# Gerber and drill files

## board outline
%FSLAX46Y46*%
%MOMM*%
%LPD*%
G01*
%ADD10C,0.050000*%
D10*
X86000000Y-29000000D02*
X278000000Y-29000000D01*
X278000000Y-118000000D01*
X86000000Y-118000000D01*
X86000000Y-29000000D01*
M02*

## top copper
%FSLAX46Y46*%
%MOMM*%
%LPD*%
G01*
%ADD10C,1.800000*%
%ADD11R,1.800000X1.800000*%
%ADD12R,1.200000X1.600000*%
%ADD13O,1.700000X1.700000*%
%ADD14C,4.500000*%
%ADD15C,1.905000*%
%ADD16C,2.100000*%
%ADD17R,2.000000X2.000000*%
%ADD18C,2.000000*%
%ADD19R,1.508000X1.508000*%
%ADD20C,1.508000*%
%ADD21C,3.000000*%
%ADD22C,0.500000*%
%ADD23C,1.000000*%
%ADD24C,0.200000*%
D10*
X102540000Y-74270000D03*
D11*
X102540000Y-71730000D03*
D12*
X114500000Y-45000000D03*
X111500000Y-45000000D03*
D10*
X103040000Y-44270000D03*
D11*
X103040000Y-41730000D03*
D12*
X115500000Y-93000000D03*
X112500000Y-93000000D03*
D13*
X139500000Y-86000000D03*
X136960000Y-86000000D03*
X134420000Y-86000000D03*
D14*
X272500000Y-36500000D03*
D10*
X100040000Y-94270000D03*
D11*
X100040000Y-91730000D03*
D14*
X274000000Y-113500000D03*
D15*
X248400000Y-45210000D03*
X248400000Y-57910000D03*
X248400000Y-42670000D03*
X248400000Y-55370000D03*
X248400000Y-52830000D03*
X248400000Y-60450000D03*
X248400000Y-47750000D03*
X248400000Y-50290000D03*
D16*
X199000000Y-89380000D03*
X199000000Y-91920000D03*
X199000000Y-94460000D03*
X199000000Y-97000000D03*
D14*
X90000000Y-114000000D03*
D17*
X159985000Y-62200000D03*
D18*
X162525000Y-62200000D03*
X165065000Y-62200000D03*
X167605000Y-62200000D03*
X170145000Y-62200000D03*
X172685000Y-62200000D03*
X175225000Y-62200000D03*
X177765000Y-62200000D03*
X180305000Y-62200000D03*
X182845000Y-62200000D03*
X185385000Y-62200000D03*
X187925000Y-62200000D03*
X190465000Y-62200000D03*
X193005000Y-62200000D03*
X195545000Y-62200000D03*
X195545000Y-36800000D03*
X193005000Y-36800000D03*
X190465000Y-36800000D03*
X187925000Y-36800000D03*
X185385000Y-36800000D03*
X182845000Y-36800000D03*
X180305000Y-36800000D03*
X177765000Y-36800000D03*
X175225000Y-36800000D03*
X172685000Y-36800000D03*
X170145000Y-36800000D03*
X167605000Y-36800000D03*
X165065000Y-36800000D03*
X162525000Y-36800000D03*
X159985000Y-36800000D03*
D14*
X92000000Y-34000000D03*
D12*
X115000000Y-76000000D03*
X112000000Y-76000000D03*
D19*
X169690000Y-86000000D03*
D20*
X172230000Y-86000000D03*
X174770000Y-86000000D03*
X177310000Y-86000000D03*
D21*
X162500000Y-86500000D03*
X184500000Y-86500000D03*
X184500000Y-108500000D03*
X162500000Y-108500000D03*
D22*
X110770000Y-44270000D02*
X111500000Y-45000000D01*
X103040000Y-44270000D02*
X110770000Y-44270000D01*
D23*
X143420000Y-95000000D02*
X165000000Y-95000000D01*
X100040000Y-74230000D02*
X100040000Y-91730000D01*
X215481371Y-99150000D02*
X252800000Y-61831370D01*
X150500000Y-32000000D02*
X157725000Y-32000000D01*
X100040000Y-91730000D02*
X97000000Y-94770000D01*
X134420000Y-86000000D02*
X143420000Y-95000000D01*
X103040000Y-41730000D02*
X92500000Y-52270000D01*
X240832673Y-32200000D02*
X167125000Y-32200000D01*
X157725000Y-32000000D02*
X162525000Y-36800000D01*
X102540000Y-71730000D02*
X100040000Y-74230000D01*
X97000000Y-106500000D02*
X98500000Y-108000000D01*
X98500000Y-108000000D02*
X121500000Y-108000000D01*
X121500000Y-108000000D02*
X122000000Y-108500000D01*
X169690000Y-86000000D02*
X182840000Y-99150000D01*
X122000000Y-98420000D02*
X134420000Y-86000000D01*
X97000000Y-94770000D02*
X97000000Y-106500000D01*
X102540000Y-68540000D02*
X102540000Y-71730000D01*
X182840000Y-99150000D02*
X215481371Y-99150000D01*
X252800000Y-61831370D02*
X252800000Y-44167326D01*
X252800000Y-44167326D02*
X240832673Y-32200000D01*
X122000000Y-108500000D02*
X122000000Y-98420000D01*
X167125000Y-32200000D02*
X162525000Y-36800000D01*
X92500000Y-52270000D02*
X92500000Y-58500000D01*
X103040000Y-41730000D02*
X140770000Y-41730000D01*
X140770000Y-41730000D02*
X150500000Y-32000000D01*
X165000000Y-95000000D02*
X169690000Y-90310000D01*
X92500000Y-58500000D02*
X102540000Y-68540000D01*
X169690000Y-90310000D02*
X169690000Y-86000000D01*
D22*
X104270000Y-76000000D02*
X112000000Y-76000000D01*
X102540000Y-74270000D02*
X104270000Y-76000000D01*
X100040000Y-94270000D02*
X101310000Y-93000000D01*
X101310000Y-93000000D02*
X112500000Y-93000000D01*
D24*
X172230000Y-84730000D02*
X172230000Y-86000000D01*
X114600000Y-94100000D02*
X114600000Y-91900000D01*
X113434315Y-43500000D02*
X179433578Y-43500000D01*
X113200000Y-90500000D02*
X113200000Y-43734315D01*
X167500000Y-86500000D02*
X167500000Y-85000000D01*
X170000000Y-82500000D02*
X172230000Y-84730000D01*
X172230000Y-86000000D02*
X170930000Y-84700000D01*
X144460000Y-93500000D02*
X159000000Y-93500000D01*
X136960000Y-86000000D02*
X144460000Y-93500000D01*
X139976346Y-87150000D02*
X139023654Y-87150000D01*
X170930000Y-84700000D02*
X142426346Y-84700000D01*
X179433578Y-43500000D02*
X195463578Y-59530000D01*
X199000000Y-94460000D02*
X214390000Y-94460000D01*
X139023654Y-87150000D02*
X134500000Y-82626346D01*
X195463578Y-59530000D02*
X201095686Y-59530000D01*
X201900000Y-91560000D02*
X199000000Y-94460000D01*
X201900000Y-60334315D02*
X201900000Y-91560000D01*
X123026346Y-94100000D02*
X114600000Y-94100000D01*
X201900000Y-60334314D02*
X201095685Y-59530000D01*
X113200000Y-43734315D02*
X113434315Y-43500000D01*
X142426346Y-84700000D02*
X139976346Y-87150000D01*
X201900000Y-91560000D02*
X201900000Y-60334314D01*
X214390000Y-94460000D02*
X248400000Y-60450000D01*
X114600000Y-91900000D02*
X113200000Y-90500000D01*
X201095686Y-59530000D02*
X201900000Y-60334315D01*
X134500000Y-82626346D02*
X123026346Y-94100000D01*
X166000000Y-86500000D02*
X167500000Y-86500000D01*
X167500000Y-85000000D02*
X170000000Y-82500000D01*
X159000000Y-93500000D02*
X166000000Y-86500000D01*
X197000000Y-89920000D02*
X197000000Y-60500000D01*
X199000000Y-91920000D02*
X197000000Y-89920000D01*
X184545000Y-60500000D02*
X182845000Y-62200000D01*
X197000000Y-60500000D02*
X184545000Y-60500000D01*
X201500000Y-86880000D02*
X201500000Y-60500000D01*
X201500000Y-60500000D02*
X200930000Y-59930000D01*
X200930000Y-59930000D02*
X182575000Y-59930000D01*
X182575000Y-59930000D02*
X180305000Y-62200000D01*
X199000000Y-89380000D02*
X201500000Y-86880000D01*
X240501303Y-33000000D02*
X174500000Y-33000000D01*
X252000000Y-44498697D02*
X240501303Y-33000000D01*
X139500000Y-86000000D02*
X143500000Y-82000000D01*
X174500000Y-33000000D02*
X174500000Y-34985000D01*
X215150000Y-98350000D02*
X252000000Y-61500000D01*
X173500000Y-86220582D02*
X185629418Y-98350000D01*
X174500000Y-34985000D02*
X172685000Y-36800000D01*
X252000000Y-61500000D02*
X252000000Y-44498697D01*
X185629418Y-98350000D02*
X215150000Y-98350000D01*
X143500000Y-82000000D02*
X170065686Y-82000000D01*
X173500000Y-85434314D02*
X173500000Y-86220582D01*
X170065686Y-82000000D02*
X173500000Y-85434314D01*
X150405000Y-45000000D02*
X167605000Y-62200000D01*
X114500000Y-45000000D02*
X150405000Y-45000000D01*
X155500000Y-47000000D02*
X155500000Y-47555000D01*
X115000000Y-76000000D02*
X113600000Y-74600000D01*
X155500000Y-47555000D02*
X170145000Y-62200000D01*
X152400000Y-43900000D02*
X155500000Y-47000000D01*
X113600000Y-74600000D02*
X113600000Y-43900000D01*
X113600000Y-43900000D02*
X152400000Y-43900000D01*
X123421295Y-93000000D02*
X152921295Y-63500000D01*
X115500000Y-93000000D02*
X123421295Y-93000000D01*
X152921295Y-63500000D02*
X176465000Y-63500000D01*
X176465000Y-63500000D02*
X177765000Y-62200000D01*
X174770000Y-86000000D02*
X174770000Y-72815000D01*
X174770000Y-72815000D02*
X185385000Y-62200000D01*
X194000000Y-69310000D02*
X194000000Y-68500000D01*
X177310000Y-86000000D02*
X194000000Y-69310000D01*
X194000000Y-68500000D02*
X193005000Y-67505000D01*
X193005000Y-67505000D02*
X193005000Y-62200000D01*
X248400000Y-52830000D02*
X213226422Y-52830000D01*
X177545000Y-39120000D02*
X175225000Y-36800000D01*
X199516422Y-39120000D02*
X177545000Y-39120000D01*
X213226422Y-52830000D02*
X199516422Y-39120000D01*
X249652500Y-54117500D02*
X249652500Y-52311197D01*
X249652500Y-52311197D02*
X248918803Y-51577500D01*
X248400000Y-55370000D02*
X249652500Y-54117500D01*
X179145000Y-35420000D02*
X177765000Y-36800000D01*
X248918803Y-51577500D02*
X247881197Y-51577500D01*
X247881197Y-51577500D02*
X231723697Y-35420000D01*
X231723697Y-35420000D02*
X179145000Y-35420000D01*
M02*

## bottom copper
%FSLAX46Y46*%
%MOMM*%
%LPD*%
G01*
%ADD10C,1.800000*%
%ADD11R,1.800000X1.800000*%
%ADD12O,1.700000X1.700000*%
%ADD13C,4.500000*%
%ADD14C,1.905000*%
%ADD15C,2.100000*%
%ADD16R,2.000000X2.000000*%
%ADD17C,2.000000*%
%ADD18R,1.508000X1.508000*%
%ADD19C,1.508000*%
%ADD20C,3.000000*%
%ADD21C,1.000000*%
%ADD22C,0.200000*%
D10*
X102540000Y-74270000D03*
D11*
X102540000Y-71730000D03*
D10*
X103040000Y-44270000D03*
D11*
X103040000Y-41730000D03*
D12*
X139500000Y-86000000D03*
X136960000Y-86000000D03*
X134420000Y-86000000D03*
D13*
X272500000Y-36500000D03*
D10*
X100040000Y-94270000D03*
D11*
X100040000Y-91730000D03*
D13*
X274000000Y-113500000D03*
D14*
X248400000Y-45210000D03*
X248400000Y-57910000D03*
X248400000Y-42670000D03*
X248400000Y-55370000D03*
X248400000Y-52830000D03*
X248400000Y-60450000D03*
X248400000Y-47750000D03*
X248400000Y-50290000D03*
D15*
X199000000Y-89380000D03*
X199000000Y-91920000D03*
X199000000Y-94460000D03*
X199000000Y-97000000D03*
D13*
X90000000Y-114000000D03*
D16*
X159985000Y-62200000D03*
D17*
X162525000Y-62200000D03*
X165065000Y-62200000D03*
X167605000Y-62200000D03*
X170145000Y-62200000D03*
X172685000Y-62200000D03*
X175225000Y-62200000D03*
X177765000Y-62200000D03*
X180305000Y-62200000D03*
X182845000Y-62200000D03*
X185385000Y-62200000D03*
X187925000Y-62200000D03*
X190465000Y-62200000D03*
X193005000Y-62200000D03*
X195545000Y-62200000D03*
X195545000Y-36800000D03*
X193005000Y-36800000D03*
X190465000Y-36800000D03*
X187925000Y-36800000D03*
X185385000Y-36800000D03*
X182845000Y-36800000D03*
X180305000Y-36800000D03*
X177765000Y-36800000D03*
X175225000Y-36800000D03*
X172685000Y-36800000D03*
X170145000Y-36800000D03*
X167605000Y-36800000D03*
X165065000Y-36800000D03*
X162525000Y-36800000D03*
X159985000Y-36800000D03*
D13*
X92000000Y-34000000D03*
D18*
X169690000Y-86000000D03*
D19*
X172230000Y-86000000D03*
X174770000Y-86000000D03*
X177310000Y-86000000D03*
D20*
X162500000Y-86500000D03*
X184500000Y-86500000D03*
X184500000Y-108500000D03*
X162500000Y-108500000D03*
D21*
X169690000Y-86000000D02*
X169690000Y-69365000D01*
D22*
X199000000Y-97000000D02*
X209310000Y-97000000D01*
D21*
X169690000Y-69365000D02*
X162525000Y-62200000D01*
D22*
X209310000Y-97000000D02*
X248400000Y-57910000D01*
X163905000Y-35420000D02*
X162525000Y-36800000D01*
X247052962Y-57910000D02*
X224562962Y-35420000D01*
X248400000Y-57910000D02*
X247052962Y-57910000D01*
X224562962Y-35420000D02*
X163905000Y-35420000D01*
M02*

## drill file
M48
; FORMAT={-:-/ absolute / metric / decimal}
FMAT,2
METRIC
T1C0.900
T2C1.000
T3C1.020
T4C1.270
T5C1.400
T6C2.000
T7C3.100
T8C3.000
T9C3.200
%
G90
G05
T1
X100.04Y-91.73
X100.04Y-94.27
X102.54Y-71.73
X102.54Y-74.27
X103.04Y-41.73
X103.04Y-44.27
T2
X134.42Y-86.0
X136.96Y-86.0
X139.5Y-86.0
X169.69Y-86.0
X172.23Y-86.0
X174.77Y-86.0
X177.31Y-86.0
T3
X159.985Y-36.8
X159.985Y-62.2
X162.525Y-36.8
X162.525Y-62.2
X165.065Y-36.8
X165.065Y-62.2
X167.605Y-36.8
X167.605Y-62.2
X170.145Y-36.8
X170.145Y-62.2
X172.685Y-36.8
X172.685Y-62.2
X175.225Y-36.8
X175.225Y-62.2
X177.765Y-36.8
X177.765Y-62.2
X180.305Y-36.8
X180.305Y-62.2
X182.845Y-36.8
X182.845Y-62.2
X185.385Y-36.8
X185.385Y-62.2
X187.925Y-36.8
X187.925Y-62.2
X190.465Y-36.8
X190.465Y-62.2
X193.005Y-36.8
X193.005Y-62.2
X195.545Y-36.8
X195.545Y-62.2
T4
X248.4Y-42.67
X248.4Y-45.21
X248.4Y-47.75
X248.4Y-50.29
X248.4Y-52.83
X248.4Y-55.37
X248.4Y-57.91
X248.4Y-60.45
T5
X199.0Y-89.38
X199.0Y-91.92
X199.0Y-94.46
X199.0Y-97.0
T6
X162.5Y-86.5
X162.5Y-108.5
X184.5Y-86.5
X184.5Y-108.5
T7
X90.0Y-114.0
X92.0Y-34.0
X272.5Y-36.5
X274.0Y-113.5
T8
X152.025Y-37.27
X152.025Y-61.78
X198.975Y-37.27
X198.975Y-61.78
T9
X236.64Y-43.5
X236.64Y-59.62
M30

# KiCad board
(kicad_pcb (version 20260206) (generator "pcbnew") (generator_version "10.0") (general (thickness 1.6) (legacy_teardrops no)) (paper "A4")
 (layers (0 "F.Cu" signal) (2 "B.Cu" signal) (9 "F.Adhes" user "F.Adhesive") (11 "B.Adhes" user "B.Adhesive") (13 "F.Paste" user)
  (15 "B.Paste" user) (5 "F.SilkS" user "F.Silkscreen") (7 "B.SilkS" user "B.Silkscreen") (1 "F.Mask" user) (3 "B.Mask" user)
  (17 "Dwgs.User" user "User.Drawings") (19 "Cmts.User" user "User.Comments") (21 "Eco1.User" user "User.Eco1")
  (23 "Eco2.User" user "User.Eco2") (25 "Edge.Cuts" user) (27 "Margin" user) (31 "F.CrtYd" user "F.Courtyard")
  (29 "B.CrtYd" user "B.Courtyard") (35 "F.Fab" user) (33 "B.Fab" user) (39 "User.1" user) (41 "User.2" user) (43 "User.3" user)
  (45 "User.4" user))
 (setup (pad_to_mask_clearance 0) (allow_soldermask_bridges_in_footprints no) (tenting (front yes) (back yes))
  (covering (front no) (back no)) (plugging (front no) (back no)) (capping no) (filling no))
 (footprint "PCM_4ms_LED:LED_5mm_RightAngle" (layer "F.Cu") (at 98 73 -90)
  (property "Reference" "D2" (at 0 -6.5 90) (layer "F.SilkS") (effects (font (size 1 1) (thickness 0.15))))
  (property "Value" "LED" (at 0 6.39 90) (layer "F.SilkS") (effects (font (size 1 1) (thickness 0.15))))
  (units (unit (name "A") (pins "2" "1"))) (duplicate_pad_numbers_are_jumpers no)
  (pad "1" thru_hole circle (at 1.27 -4.54 270) (size 1.8 1.8) (drill 0.9) (layers "*.Cu" "*.Mask") (remove_unused_layers no)
   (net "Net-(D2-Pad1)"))
  (pad "2" thru_hole rect (at -1.27 -4.54 270) (size 1.8 1.8) (drill 0.9) (layers "*.Cu" "*.Mask") (remove_unused_layers no) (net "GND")))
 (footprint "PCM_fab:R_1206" (layer "F.Cu") (at 113 45 180)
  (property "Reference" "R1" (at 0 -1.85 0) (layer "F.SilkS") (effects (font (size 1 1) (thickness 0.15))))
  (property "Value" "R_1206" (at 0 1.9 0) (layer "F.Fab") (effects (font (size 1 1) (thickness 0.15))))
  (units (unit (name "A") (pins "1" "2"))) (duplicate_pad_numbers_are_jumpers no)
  (pad "1" smd rect (at -1.5 0 180) (size 1.2 1.6) (layers "F.Cu" "F.Mask" "F.Paste") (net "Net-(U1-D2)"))
  (pad "2" smd rect (at 1.5 0 180) (size 1.2 1.6) (layers "F.Cu" "F.Mask" "F.Paste") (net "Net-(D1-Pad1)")))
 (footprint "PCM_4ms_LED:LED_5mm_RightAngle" (layer "F.Cu") (at 98.5 43 -90)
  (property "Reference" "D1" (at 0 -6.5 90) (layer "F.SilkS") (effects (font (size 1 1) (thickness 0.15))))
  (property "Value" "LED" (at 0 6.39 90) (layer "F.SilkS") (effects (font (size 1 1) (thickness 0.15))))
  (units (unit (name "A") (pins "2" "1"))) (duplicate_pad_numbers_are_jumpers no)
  (pad "1" thru_hole circle (at 1.27 -4.54 270) (size 1.8 1.8) (drill 0.9) (layers "*.Cu" "*.Mask") (remove_unused_layers no)
   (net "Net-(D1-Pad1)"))
  (pad "2" thru_hole rect (at -1.27 -4.54 270) (size 1.8 1.8) (drill 0.9) (layers "*.Cu" "*.Mask") (remove_unused_layers no) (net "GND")))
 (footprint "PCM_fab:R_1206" (layer "F.Cu") (at 114 93 180)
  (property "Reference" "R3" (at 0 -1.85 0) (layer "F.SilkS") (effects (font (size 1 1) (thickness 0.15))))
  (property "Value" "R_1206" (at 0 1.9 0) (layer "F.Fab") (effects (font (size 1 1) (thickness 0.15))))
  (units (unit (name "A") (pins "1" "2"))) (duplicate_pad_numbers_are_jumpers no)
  (pad "1" smd rect (at -1.5 0 180) (size 1.2 1.6) (layers "F.Cu" "F.Mask" "F.Paste") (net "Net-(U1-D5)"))
  (pad "2" smd rect (at 1.5 0 180) (size 1.2 1.6) (layers "F.Cu" "F.Mask" "F.Paste") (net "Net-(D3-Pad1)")))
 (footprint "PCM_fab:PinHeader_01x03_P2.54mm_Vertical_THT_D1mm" (layer "F.Cu") (at 139.5 86 -90)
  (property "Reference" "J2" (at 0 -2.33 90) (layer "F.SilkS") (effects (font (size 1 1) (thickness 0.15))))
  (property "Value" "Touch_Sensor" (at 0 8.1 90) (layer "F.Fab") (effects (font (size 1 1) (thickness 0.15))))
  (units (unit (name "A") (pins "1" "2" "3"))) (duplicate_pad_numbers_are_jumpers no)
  (pad "1" thru_hole oval (at 0 0 270) (size 1.7 1.7) (drill 1) (layers "*.Cu" "*.Mask") (remove_unused_layers no) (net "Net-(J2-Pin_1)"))
  (pad "2" thru_hole oval (at 0 2.54 270) (size 1.7 1.7) (drill 1) (layers "*.Cu" "*.Mask") (remove_unused_layers no) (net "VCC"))
  (pad "3" thru_hole oval (at 0 5.08 270) (size 1.7 1.7) (drill 1) (layers "*.Cu" "*.Mask") (remove_unused_layers no) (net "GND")))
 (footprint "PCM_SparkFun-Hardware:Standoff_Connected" (layer "F.Cu") (at 272.5 36.5)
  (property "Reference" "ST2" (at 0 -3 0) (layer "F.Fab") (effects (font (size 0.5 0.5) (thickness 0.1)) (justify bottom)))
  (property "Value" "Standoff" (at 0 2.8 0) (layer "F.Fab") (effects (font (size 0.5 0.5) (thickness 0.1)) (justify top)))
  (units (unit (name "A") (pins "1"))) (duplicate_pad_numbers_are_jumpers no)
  (pad "1" thru_hole circle (at 0 0) (size 4.5 4.5) (drill 3.1) (layers "*.Cu" "*.Mask") (remove_unused_layers no)
   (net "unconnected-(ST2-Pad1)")))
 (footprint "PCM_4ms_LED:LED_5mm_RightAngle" (layer "F.Cu") (at 95.5 93 -90)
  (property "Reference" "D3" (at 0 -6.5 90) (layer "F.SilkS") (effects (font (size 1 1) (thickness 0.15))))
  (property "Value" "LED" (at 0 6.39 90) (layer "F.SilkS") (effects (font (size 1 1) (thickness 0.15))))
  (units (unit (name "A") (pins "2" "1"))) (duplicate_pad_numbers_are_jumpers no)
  (pad "1" thru_hole circle (at 1.27 -4.54 270) (size 1.8 1.8) (drill 0.9) (layers "*.Cu" "*.Mask") (remove_unused_layers no)
   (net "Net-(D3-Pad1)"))
  (pad "2" thru_hole rect (at -1.27 -4.54 270) (size 1.8 1.8) (drill 0.9) (layers "*.Cu" "*.Mask") (remove_unused_layers no) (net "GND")))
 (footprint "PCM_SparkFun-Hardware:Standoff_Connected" (layer "F.Cu") (at 274 113.5)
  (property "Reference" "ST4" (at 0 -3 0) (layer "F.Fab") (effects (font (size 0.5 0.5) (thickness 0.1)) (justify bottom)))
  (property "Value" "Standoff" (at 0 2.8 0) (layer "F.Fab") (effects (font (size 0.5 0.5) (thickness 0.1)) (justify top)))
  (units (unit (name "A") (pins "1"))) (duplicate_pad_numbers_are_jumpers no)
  (pad "1" thru_hole circle (at 0 0) (size 4.5 4.5) (drill 3.1) (layers "*.Cu" "*.Mask") (remove_unused_layers no)
   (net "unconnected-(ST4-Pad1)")))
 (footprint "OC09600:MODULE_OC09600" (layer "F.Cu") (at 242.07 51.56 180)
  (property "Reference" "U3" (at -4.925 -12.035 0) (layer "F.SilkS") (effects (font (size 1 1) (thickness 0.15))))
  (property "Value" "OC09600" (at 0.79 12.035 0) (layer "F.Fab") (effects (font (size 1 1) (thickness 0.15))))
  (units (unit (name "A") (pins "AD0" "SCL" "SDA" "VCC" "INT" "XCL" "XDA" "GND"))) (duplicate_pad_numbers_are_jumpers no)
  (pad "" np_thru_hole circle (at 5.43 -8.06 180) (size 3.2 3.2) (drill 3.2) (layers "*.Cu" "*.Mask"))
  (pad "" np_thru_hole circle (at 5.43 8.06 180) (size 3.2 3.2) (drill 3.2) (layers "*.Cu" "*.Mask"))
  (pad "AD0" thru_hole circle (at -6.33 6.35 180) (size 1.905 1.905) (drill 1.27) (layers "*.Cu" "*.Mask") (remove_unused_layers no)
   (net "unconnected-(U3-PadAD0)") (solder_mask_margin 0.102))
  (pad "GND" thru_hole circle (at -6.33 -6.35 180) (size 1.905 1.905) (drill 1.27) (layers "*.Cu" "*.Mask") (remove_unused_layers no)
   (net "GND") (solder_mask_margin 0.102))
  (pad "INT" thru_hole circle (at -6.33 8.89 180) (size 1.905 1.905) (drill 1.27) (layers "*.Cu" "*.Mask") (remove_unused_layers no)
   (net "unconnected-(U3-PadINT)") (solder_mask_margin 0.102))
  (pad "SCL" thru_hole circle (at -6.33 -3.81 180) (size 1.905 1.905) (drill 1.27) (layers "*.Cu" "*.Mask") (remove_unused_layers no)
   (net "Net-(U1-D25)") (solder_mask_margin 0.102))
  (pad "SDA" thru_hole circle (at -6.33 -1.27 180) (size 1.905 1.905) (drill 1.27) (layers "*.Cu" "*.Mask") (remove_unused_layers no)
   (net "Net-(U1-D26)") (solder_mask_margin 0.102))
  (pad "VCC" thru_hole circle (at -6.33 -8.89 180) (size 1.905 1.905) (drill 1.27) (layers "*.Cu" "*.Mask") (remove_unused_layers no)
   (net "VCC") (solder_mask_margin 0.102))
  (pad "XCL" thru_hole circle (at -6.33 3.81 180) (size 1.905 1.905) (drill 1.27) (layers "*.Cu" "*.Mask") (remove_unused_layers no)
   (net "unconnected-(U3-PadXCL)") (solder_mask_margin 0.102))
  (pad "XDA" thru_hole circle (at -6.33 1.27 180) (size 1.905 1.905) (drill 1.27) (layers "*.Cu" "*.Mask") (remove_unused_layers no)
   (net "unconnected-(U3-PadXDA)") (solder_mask_margin 0.102)))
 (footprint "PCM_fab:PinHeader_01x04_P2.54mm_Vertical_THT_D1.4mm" (layer "F.Cu") (at 199 89.38)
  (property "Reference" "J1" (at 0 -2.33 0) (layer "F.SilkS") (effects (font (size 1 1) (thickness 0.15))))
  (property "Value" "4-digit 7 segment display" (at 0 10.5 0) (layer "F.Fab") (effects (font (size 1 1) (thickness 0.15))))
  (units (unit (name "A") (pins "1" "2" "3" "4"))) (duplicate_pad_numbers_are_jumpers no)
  (pad "1" thru_hole circle (at 0 0) (size 2.1 2.1) (drill 1.4) (layers "*.Cu" "*.Mask") (remove_unused_layers no) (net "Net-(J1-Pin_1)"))
  (pad "2" thru_hole circle (at 0 2.54) (size 2.1 2.1) (drill 1.4) (layers "*.Cu" "*.Mask") (remove_unused_layers no) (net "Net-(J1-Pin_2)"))
  (pad "3" thru_hole circle (at 0 5.08) (size 2.1 2.1) (drill 1.4) (layers "*.Cu" "*.Mask") (remove_unused_layers no) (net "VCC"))
  (pad "4" thru_hole circle (at 0 7.62) (size 2.1 2.1) (drill 1.4) (layers "*.Cu" "*.Mask") (remove_unused_layers no) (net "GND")))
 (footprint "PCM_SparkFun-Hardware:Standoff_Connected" (layer "F.Cu") (at 90 114)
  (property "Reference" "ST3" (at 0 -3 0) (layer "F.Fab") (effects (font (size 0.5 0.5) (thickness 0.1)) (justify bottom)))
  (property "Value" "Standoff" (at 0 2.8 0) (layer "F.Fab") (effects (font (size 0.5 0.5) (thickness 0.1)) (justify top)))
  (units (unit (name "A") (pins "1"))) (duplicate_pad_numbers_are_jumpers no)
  (pad "1" thru_hole circle (at 0 0) (size 4.5 4.5) (drill 3.1) (layers "*.Cu" "*.Mask") (remove_unused_layers no)
   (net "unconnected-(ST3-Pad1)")))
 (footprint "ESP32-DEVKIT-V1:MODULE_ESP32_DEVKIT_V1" (layer "F.Cu") (at 175.5 49.5 90)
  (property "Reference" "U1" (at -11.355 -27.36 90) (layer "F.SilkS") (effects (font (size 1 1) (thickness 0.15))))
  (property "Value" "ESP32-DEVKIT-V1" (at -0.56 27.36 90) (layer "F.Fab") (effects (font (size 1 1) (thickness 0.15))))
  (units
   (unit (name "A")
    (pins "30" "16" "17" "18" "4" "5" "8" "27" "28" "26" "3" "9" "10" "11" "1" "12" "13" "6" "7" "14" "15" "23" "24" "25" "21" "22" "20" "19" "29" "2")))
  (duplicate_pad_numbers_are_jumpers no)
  (pad "" np_thru_hole circle (at -12.28 -23.475 90) (size 3 3) (drill 3) (layers "*.Cu" "*.Mask"))
  (pad "" np_thru_hole circle (at -12.28 23.475 90) (size 3 3) (drill 3) (layers "*.Cu" "*.Mask"))
  (pad "" np_thru_hole circle (at 12.23 -23.475 90) (size 3 3) (drill 3) (layers "*.Cu" "*.Mask"))
  (pad "" np_thru_hole circle (at 12.23 23.475 90) (size 3 3) (drill 3) (layers "*.Cu" "*.Mask"))
  (pad "1" thru_hole rect (at -12.7 -15.515 90) (size 2 2) (drill 1.02) (layers "*.Cu" "*.Mask") (remove_unused_layers no) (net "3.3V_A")
   (solder_mask_margin 0.102))
  (pad "2" thru_hole circle (at -12.7 -12.975 90) (size 2 2) (drill 1.02) (layers "*.Cu" "*.Mask") (remove_unused_layers no) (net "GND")
   (solder_mask_margin 0.102))
  (pad "3" thru_hole circle (at -12.7 -10.435 90) (size 2 2) (drill 1.02) (layers "*.Cu" "*.Mask") (remove_unused_layers no)
   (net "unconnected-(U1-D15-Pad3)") (solder_mask_margin 0.102))
  (pad "4" thru_hole circle (at -12.7 -7.895 90) (size 2 2) (drill 1.02) (layers "*.Cu" "*.Mask") (remove_unused_layers no)
   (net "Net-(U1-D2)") (solder_mask_margin 0.102))
  (pad "5" thru_hole circle (at -12.7 -5.355 90) (size 2 2) (drill 1.02) (layers "*.Cu" "*.Mask") (remove_unused_layers no)
   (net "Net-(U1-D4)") (solder_mask_margin 0.102))
  (pad "6" thru_hole circle (at -12.7 -2.815 90) (size 2 2) (drill 1.02) (layers "*.Cu" "*.Mask") (remove_unused_layers no)
   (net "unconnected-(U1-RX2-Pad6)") (solder_mask_margin 0.102))
  (pad "7" thru_hole circle (at -12.7 -0.275 90) (size 2 2) (drill 1.02) (layers "*.Cu" "*.Mask") (remove_unused_layers no)
   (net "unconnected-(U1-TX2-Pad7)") (solder_mask_margin 0.102))
  (pad "8" thru_hole circle (at -12.7 2.265 90) (size 2 2) (drill 1.02) (layers "*.Cu" "*.Mask") (remove_unused_layers no)
   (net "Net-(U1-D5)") (solder_mask_margin 0.102))
  (pad "9" thru_hole circle (at -12.7 4.805 90) (size 2 2) (drill 1.02) (layers "*.Cu" "*.Mask") (remove_unused_layers no)
   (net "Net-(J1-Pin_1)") (solder_mask_margin 0.102))
  (pad "10" thru_hole circle (at -12.7 7.345 90) (size 2 2) (drill 1.02) (layers "*.Cu" "*.Mask") (remove_unused_layers no)
   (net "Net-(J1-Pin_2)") (solder_mask_margin 0.102))
  (pad "11" thru_hole circle (at -12.7 9.885 90) (size 2 2) (drill 1.02) (layers "*.Cu" "*.Mask") (remove_unused_layers no) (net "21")
   (solder_mask_margin 0.102))
  (pad "12" thru_hole circle (at -12.7 12.425 90) (size 2 2) (drill 1.02) (layers "*.Cu" "*.Mask") (remove_unused_layers no)
   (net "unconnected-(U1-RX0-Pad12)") (solder_mask_margin 0.102))
  (pad "13" thru_hole circle (at -12.7 14.965 90) (size 2 2) (drill 1.02) (layers "*.Cu" "*.Mask") (remove_unused_layers no)
   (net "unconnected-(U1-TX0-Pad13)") (solder_mask_margin 0.102))
  (pad "14" thru_hole circle (at -12.7 17.505 90) (size 2 2) (drill 1.02) (layers "*.Cu" "*.Mask") (remove_unused_layers no) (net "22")
   (solder_mask_margin 0.102))
  (pad "15" thru_hole circle (at -12.7 20.045 90) (size 2 2) (drill 1.02) (layers "*.Cu" "*.Mask") (remove_unused_layers no)
   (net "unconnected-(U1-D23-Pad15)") (solder_mask_margin 0.102))
  (pad "16" thru_hole circle (at 12.7 20.045 90) (size 2 2) (drill 1.02) (layers "*.Cu" "*.Mask") (remove_unused_layers no)
   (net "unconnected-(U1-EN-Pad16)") (solder_mask_margin 0.102))
  (pad "17" thru_hole circle (at 12.7 17.505 90) (size 2 2) (drill 1.02) (layers "*.Cu" "*.Mask") (remove_unused_layers no)
   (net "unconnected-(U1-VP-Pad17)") (solder_mask_margin 0.102))
  (pad "18" thru_hole circle (at 12.7 14.965 90) (size 2 2) (drill 1.02) (layers "*.Cu" "*.Mask") (remove_unused_layers no)
   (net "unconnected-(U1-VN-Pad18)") (solder_mask_margin 0.102))
  (pad "19" thru_hole circle (at 12.7 12.425 90) (size 2 2) (drill 1.02) (layers "*.Cu" "*.Mask") (remove_unused_layers no)
   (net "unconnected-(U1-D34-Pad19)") (solder_mask_margin 0.102))
  (pad "20" thru_hole circle (at 12.7 9.885 90) (size 2 2) (drill 1.02) (layers "*.Cu" "*.Mask") (remove_unused_layers no)
   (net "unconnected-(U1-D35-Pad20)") (solder_mask_margin 0.102))
  (pad "21" thru_hole circle (at 12.7 7.345 90) (size 2 2) (drill 1.02) (layers "*.Cu" "*.Mask") (remove_unused_layers no)
   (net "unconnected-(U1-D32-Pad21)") (solder_mask_margin 0.102))
  (pad "22" thru_hole circle (at 12.7 4.805 90) (size 2 2) (drill 1.02) (layers "*.Cu" "*.Mask") (remove_unused_layers no)
   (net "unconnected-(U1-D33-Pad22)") (solder_mask_margin 0.102))
  (pad "23" thru_hole circle (at 12.7 2.265 90) (size 2 2) (drill 1.02) (layers "*.Cu" "*.Mask") (remove_unused_layers no)
   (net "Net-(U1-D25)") (solder_mask_margin 0.102))
  (pad "24" thru_hole circle (at 12.7 -0.275 90) (size 2 2) (drill 1.02) (layers "*.Cu" "*.Mask") (remove_unused_layers no)
   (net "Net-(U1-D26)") (solder_mask_margin 0.102))
  (pad "25" thru_hole circle (at 12.7 -2.815 90) (size 2 2) (drill 1.02) (layers "*.Cu" "*.Mask") (remove_unused_layers no)
   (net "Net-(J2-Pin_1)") (solder_mask_margin 0.102))
  (pad "26" thru_hole circle (at 12.7 -5.355 90) (size 2 2) (drill 1.02) (layers "*.Cu" "*.Mask") (remove_unused_layers no)
   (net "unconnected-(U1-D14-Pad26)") (solder_mask_margin 0.102))
  (pad "27" thru_hole circle (at 12.7 -7.895 90) (size 2 2) (drill 1.02) (layers "*.Cu" "*.Mask") (remove_unused_layers no)
   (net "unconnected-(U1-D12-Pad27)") (solder_mask_margin 0.102))
  (pad "28" thru_hole circle (at 12.7 -10.435 90) (size 2 2) (drill 1.02) (layers "*.Cu" "*.Mask") (remove_unused_layers no)
   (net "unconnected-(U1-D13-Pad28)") (solder_mask_margin 0.102))
  (pad "29" thru_hole circle (at 12.7 -12.975 90) (size 2 2) (drill 1.02) (layers "*.Cu" "*.Mask") (remove_unused_layers no) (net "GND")
   (solder_mask_margin 0.102))
  (pad "30" thru_hole circle (at 12.7 -15.515 90) (size 2 2) (drill 1.02) (layers "*.Cu" "*.Mask") (remove_unused_layers no) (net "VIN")
   (solder_mask_margin 0.102))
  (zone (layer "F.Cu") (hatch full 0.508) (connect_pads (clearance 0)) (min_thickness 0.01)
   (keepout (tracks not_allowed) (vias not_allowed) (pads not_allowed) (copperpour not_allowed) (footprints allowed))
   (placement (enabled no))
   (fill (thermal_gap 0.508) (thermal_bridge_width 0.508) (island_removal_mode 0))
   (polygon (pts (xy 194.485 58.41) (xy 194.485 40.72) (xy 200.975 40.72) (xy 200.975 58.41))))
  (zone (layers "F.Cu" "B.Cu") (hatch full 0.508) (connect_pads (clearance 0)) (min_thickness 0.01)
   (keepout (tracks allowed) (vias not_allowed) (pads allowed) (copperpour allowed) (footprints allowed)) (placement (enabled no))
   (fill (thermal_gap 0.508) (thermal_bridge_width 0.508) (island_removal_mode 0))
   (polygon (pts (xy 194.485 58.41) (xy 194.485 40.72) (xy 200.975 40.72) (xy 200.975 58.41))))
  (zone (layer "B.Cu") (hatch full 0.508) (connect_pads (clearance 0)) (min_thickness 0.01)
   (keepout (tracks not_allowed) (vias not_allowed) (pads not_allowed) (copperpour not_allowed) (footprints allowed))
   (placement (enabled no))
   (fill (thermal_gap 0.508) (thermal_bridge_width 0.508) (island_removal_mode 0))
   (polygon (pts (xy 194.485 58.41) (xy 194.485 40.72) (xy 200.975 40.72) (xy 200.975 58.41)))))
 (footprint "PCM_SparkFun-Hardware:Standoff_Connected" (layer "F.Cu") (at 92 34)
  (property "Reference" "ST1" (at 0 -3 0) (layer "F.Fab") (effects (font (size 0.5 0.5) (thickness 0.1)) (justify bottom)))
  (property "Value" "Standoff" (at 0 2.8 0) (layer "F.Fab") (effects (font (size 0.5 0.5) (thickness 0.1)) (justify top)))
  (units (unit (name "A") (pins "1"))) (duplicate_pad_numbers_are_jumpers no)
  (pad "1" thru_hole circle (at 0 0) (size 4.5 4.5) (drill 3.1) (layers "*.Cu" "*.Mask") (remove_unused_layers no)
   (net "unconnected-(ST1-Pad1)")))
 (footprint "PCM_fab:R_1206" (layer "F.Cu") (at 113.5 76 180)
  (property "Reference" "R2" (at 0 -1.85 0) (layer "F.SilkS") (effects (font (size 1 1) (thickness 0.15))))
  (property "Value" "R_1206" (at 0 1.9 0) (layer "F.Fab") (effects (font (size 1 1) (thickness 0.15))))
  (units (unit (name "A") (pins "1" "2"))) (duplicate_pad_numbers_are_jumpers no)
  (pad "1" smd rect (at -1.5 0 180) (size 1.2 1.6) (layers "F.Cu" "F.Mask" "F.Paste") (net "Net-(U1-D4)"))
  (pad "2" smd rect (at 1.5 0 180) (size 1.2 1.6) (layers "F.Cu" "F.Mask" "F.Paste") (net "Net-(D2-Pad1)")))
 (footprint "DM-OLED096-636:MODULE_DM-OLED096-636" (layer "F.Cu") (at 173.5 97.5)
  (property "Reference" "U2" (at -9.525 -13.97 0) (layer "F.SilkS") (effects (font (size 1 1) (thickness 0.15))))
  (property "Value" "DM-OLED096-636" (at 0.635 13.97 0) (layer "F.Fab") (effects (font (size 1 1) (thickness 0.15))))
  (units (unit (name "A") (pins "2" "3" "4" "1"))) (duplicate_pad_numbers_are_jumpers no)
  (pad "1" thru_hole rect (at -3.81 -11.5) (size 1.508 1.508) (drill 1) (layers "*.Cu" "*.Mask") (remove_unused_layers no) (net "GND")
   (solder_mask_margin 0.102))
  (pad "2" thru_hole circle (at -1.27 -11.5) (size 1.508 1.508) (drill 1) (layers "*.Cu" "*.Mask") (remove_unused_layers no) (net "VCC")
   (solder_mask_margin 0.102))
  (pad "3" thru_hole circle (at 1.27 -11.5) (size 1.508 1.508) (drill 1) (layers "*.Cu" "*.Mask") (remove_unused_layers no) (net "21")
   (solder_mask_margin 0.102))
  (pad "4" thru_hole circle (at 3.81 -11.5) (size 1.508 1.508) (drill 1) (layers "*.Cu" "*.Mask") (remove_unused_layers no) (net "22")
   (solder_mask_margin 0.102))
  (pad "S1" thru_hole circle (at -11 -11) (size 3 3) (drill 2) (layers "*.Cu" "*.Mask") (remove_unused_layers no) (solder_mask_margin 0.102))
  (pad "S2" thru_hole circle (at 11 -11) (size 3 3) (drill 2) (layers "*.Cu" "*.Mask") (remove_unused_layers no) (solder_mask_margin 0.102))
  (pad "S3" thru_hole circle (at 11 11) (size 3 3) (drill 2) (layers "*.Cu" "*.Mask") (remove_unused_layers no) (solder_mask_margin 0.102))
  (pad "S4" thru_hole circle (at -11 11) (size 3 3) (drill 2) (layers "*.Cu" "*.Mask") (remove_unused_layers no) (solder_mask_margin 0.102)))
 (gr_rect (start 86 29) (end 278 118) (stroke (width 0.05) (type default)) (fill no) (layer "Edge.Cuts"))
 (segment (start 110.77 44.27) (end 111.5 45) (width 0.5) (layer "F.Cu") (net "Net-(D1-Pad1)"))
 (segment (start 103.04 44.27) (end 110.77 44.27) (width 0.5) (layer "F.Cu") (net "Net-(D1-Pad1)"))
 (segment (start 143.42 95) (end 165 95) (width 1) (layer "F.Cu") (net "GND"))
 (segment (start 100.04 74.23) (end 100.04 91.73) (width 1) (layer "F.Cu") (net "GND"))
 (segment (start 215.481371 99.15) (end 252.8 61.83137) (width 1) (layer "F.Cu") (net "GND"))
 (segment (start 150.5 32) (end 157.725 32) (width 1) (layer "F.Cu") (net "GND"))
 (segment (start 100.04 91.73) (end 97 94.77) (width 1) (layer "F.Cu") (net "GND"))
 (segment (start 134.42 86) (end 143.42 95) (width 1) (layer "F.Cu") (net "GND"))
 (segment (start 103.04 41.73) (end 92.5 52.27) (width 1) (layer "F.Cu") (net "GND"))
 (segment (start 240.832673 32.2) (end 167.125 32.2) (width 1) (layer "F.Cu") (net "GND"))
 (segment (start 157.725 32) (end 162.525 36.8) (width 1) (layer "F.Cu") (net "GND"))
 (segment (start 102.54 71.73) (end 100.04 74.23) (width 1) (layer "F.Cu") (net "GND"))
 (segment (start 97 106.5) (end 98.5 108) (width 1) (layer "F.Cu") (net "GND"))
 (segment (start 98.5 108) (end 121.5 108) (width 1) (layer "F.Cu") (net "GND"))
 (segment (start 121.5 108) (end 122 108.5) (width 1) (layer "F.Cu") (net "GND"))
 (segment (start 169.69 86) (end 182.84 99.15) (width 1) (layer "F.Cu") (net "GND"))
 (segment (start 122 98.42) (end 134.42 86) (width 1) (layer "F.Cu") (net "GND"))
 (segment (start 97 94.77) (end 97 106.5) (width 1) (layer "F.Cu") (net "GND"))
 (segment (start 102.54 68.54) (end 102.54 71.73) (width 1) (layer "F.Cu") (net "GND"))
 (segment (start 182.84 99.15) (end 215.481371 99.15) (width 1) (layer "F.Cu") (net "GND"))
 (segment (start 252.8 61.83137) (end 252.8 44.167326) (width 1) (layer "F.Cu") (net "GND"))
 (segment (start 252.8 44.167326) (end 240.832673 32.2) (width 1) (layer "F.Cu") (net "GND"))
 (segment (start 122 108.5) (end 122 98.42) (width 1) (layer "F.Cu") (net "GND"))
 (segment (start 167.125 32.2) (end 162.525 36.8) (width 1) (layer "F.Cu") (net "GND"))
 (segment (start 92.5 52.27) (end 92.5 58.5) (width 1) (layer "F.Cu") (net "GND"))
 (segment (start 103.04 41.73) (end 140.77 41.73) (width 1) (layer "F.Cu") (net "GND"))
 (segment (start 140.77 41.73) (end 150.5 32) (width 1) (layer "F.Cu") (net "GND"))
 (segment (start 165 95) (end 169.69 90.31) (width 1) (layer "F.Cu") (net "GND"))
 (segment (start 92.5 58.5) (end 102.54 68.54) (width 1) (layer "F.Cu") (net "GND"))
 (segment (start 169.69 90.31) (end 169.69 86) (width 1) (layer "F.Cu") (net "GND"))
 (segment (start 169.69 86) (end 169.69 69.365) (width 1) (layer "B.Cu") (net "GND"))
 (segment (start 199 97) (end 209.31 97) (width 0.2) (layer "B.Cu") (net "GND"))
 (segment (start 169.69 69.365) (end 162.525 62.2) (width 1) (layer "B.Cu") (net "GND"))
 (segment (start 209.31 97) (end 248.4 57.91) (width 0.2) (layer "B.Cu") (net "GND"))
 (segment (start 163.905 35.42) (end 162.525 36.8) (width 0.2) (layer "B.Cu") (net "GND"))
 (segment (start 247.052962 57.91) (end 224.562962 35.42) (width 0.2) (layer "B.Cu") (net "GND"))
 (segment (start 248.4 57.91) (end 247.052962 57.91) (width 0.2) (layer "B.Cu") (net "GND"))
 (segment (start 224.562962 35.42) (end 163.905 35.42) (width 0.2) (layer "B.Cu") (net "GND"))
 (segment (start 104.27 76) (end 112 76) (width 0.5) (layer "F.Cu") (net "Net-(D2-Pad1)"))
 (segment (start 102.54 74.27) (end 104.27 76) (width 0.5) (layer "F.Cu") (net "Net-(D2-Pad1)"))
 (segment (start 100.04 94.27) (end 101.31 93) (width 0.5) (layer "F.Cu") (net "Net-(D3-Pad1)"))
 (segment (start 101.31 93) (end 112.5 93) (width 0.5) (layer "F.Cu") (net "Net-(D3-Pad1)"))
 (segment (start 172.23 84.73) (end 172.23 86) (width 0.2) (layer "F.Cu") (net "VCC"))
 (segment (start 114.6 94.1) (end 114.6 91.9) (width 0.2) (layer "F.Cu") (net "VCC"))
 (segment (start 113.434315 43.5) (end 179.433578 43.5) (width 0.2) (layer "F.Cu") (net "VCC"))
 (segment (start 113.2 90.5) (end 113.2 43.734315) (width 0.2) (layer "F.Cu") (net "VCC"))
 (segment (start 167.5 86.5) (end 167.5 85) (width 0.2) (layer "F.Cu") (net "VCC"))
 (segment (start 170 82.5) (end 172.23 84.73) (width 0.2) (layer "F.Cu") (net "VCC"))
 (segment (start 172.23 86) (end 170.93 84.7) (width 0.2) (layer "F.Cu") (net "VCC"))
 (segment (start 144.46 93.5) (end 159 93.5) (width 0.2) (layer "F.Cu") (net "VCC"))
 (segment (start 136.96 86) (end 144.46 93.5) (width 0.2) (layer "F.Cu") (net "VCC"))
 (segment (start 139.976346 87.15) (end 139.023654 87.15) (width 0.2) (layer "F.Cu") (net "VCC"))
 (segment (start 170.93 84.7) (end 142.426346 84.7) (width 0.2) (layer "F.Cu") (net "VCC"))
 (segment (start 179.433578 43.5) (end 195.463578 59.53) (width 0.2) (layer "F.Cu") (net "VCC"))
 (segment (start 199 94.46) (end 214.39 94.46) (width 0.2) (layer "F.Cu") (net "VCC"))
 (segment (start 139.023654 87.15) (end 134.5 82.626346) (width 0.2) (layer "F.Cu") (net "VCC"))
 (segment (start 195.463578 59.53) (end 201.095686 59.53) (width 0.2) (layer "F.Cu") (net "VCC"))
 (segment (start 201.9 91.56) (end 199 94.46) (width 0.2) (layer "F.Cu") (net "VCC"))
 (segment (start 201.9 60.334315) (end 201.9 91.56) (width 0.2) (layer "F.Cu") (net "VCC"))
 (segment (start 123.026346 94.1) (end 114.6 94.1) (width 0.2) (layer "F.Cu") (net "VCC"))
 (segment (start 201.9 60.334314) (end 201.095685 59.53) (width 0.2) (layer "F.Cu") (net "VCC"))
 (segment (start 113.2 43.734315) (end 113.434315 43.5) (width 0.2) (layer "F.Cu") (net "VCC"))
 (segment (start 142.426346 84.7) (end 139.976346 87.15) (width 0.2) (layer "F.Cu") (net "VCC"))
 (segment (start 201.9 91.56) (end 201.9 60.334314) (width 0.2) (layer "F.Cu") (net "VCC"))
 (segment (start 214.39 94.46) (end 248.4 60.45) (width 0.2) (layer "F.Cu") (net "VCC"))
 (segment (start 114.6 91.9) (end 113.2 90.5) (width 0.2) (layer "F.Cu") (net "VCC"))
 (segment (start 201.095686 59.53) (end 201.9 60.334315) (width 0.2) (layer "F.Cu") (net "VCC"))
 (segment (start 134.5 82.626346) (end 123.026346 94.1) (width 0.2) (layer "F.Cu") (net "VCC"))
 (segment (start 166 86.5) (end 167.5 86.5) (width 0.2) (layer "F.Cu") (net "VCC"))
 (segment (start 167.5 85) (end 170 82.5) (width 0.2) (layer "F.Cu") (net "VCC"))
 (segment (start 159 93.5) (end 166 86.5) (width 0.2) (layer "F.Cu") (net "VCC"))
 (segment (start 197 89.92) (end 197 60.5) (width 0.2) (layer "F.Cu") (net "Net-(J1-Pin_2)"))
 (segment (start 199 91.92) (end 197 89.92) (width 0.2) (layer "F.Cu") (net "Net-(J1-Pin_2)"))
 (segment (start 184.545 60.5) (end 182.845 62.2) (width 0.2) (layer "F.Cu") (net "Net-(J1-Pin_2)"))
 (segment (start 197 60.5) (end 184.545 60.5) (width 0.2) (layer "F.Cu") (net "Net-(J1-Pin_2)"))
 (segment (start 201.5 86.88) (end 201.5 60.5) (width 0.2) (layer "F.Cu") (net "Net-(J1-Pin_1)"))
 (segment (start 201.5 60.5) (end 200.93 59.93) (width 0.2) (layer "F.Cu") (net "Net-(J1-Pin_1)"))
 (segment (start 200.93 59.93) (end 182.575 59.93) (width 0.2) (layer "F.Cu") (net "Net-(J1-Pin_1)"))
 (segment (start 182.575 59.93) (end 180.305 62.2) (width 0.2) (layer "F.Cu") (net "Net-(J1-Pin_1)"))
 (segment (start 199 89.38) (end 201.5 86.88) (width 0.2) (layer "F.Cu") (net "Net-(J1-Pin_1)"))
 (segment (start 240.501303 33) (end 174.5 33) (width 0.2) (layer "F.Cu") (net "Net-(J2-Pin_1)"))
 (segment (start 252 44.498697) (end 240.501303 33) (width 0.2) (layer "F.Cu") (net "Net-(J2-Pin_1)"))
 (segment (start 139.5 86) (end 143.5 82) (width 0.2) (layer "F.Cu") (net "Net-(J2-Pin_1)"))
 (segment (start 174.5 33) (end 174.5 34.985) (width 0.2) (layer "F.Cu") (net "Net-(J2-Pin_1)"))
 (segment (start 215.15 98.35) (end 252 61.5) (width 0.2) (layer "F.Cu") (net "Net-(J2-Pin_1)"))
 (segment (start 173.5 86.220582) (end 185.629418 98.35) (width 0.2) (layer "F.Cu") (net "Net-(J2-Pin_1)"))
 (segment (start 174.5 34.985) (end 172.685 36.8) (width 0.2) (layer "F.Cu") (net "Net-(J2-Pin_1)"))
 (segment (start 252 61.5) (end 252 44.498697) (width 0.2) (layer "F.Cu") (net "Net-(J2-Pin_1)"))
 (segment (start 185.629418 98.35) (end 215.15 98.35) (width 0.2) (layer "F.Cu") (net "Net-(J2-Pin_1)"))
 (segment (start 143.5 82) (end 170.065686 82) (width 0.2) (layer "F.Cu") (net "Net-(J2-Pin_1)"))
 (segment (start 173.5 85.434314) (end 173.5 86.220582) (width 0.2) (layer "F.Cu") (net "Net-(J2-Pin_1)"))
 (segment (start 170.065686 82) (end 173.5 85.434314) (width 0.2) (layer "F.Cu") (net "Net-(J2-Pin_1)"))
 (segment (start 150.405 45) (end 167.605 62.2) (width 0.2) (layer "F.Cu") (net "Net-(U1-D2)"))
 (segment (start 114.5 45) (end 150.405 45) (width 0.2) (layer "F.Cu") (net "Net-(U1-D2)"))
 (segment (start 155.5 47) (end 155.5 47.555) (width 0.2) (layer "F.Cu") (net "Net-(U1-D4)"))
 (segment (start 115 76) (end 113.6 74.6) (width 0.2) (layer "F.Cu") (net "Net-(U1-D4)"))
 (segment (start 155.5 47.555) (end 170.145 62.2) (width 0.2) (layer "F.Cu") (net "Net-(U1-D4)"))
 (segment (start 152.4 43.9) (end 155.5 47) (width 0.2) (layer "F.Cu") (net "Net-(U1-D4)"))
 (segment (start 113.6 74.6) (end 113.6 43.9) (width 0.2) (layer "F.Cu") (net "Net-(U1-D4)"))
 (segment (start 113.6 43.9) (end 152.4 43.9) (width 0.2) (layer "F.Cu") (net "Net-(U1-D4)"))
 (segment (start 123.421295 93) (end 152.921295 63.5) (width 0.2) (layer "F.Cu") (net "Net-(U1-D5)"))
 (segment (start 115.5 93) (end 123.421295 93) (width 0.2) (layer "F.Cu") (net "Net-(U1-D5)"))
 (segment (start 152.921295 63.5) (end 176.465 63.5) (width 0.2) (layer "F.Cu") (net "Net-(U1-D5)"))
 (segment (start 176.465 63.5) (end 177.765 62.2) (width 0.2) (layer "F.Cu") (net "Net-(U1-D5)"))
 (segment (start 174.77 86) (end 174.77 72.815) (width 0.2) (layer "F.Cu") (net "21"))
 (segment (start 174.77 72.815) (end 185.385 62.2) (width 0.2) (layer "F.Cu") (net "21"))
 (segment (start 194 69.31) (end 194 68.5) (width 0.2) (layer "F.Cu") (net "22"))
 (segment (start 177.31 86) (end 194 69.31) (width 0.2) (layer "F.Cu") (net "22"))
 (segment (start 194 68.5) (end 193.005 67.505) (width 0.2) (layer "F.Cu") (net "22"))
 (segment (start 193.005 67.505) (end 193.005 62.2) (width 0.2) (layer "F.Cu") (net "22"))
 (segment (start 248.4 52.83) (end 213.226422 52.83) (width 0.2) (layer "F.Cu") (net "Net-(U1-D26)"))
 (segment (start 177.545 39.12) (end 175.225 36.8) (width 0.2) (layer "F.Cu") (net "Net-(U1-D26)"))
 (segment (start 199.516422 39.12) (end 177.545 39.12) (width 0.2) (layer "F.Cu") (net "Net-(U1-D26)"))
 (segment (start 213.226422 52.83) (end 199.516422 39.12) (width 0.2) (layer "F.Cu") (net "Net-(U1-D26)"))
 (segment (start 249.6525 54.1175) (end 249.6525 52.311197) (width 0.2) (layer "F.Cu") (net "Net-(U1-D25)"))
 (segment (start 249.6525 52.311197) (end 248.918803 51.5775) (width 0.2) (layer "F.Cu") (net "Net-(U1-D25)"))
 (segment (start 248.4 55.37) (end 249.6525 54.1175) (width 0.2) (layer "F.Cu") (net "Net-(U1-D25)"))
 (segment (start 179.145 35.42) (end 177.765 36.8) (width 0.2) (layer "F.Cu") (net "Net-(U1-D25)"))
 (segment (start 248.918803 51.5775) (end 247.881197 51.5775) (width 0.2) (layer "F.Cu") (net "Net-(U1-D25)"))
 (segment (start 247.881197 51.5775) (end 231.723697 35.42) (width 0.2) (layer "F.Cu") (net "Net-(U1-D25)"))
 (segment (start 231.723697 35.42) (end 179.145 35.42) (width 0.2) (layer "F.Cu") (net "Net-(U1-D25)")))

